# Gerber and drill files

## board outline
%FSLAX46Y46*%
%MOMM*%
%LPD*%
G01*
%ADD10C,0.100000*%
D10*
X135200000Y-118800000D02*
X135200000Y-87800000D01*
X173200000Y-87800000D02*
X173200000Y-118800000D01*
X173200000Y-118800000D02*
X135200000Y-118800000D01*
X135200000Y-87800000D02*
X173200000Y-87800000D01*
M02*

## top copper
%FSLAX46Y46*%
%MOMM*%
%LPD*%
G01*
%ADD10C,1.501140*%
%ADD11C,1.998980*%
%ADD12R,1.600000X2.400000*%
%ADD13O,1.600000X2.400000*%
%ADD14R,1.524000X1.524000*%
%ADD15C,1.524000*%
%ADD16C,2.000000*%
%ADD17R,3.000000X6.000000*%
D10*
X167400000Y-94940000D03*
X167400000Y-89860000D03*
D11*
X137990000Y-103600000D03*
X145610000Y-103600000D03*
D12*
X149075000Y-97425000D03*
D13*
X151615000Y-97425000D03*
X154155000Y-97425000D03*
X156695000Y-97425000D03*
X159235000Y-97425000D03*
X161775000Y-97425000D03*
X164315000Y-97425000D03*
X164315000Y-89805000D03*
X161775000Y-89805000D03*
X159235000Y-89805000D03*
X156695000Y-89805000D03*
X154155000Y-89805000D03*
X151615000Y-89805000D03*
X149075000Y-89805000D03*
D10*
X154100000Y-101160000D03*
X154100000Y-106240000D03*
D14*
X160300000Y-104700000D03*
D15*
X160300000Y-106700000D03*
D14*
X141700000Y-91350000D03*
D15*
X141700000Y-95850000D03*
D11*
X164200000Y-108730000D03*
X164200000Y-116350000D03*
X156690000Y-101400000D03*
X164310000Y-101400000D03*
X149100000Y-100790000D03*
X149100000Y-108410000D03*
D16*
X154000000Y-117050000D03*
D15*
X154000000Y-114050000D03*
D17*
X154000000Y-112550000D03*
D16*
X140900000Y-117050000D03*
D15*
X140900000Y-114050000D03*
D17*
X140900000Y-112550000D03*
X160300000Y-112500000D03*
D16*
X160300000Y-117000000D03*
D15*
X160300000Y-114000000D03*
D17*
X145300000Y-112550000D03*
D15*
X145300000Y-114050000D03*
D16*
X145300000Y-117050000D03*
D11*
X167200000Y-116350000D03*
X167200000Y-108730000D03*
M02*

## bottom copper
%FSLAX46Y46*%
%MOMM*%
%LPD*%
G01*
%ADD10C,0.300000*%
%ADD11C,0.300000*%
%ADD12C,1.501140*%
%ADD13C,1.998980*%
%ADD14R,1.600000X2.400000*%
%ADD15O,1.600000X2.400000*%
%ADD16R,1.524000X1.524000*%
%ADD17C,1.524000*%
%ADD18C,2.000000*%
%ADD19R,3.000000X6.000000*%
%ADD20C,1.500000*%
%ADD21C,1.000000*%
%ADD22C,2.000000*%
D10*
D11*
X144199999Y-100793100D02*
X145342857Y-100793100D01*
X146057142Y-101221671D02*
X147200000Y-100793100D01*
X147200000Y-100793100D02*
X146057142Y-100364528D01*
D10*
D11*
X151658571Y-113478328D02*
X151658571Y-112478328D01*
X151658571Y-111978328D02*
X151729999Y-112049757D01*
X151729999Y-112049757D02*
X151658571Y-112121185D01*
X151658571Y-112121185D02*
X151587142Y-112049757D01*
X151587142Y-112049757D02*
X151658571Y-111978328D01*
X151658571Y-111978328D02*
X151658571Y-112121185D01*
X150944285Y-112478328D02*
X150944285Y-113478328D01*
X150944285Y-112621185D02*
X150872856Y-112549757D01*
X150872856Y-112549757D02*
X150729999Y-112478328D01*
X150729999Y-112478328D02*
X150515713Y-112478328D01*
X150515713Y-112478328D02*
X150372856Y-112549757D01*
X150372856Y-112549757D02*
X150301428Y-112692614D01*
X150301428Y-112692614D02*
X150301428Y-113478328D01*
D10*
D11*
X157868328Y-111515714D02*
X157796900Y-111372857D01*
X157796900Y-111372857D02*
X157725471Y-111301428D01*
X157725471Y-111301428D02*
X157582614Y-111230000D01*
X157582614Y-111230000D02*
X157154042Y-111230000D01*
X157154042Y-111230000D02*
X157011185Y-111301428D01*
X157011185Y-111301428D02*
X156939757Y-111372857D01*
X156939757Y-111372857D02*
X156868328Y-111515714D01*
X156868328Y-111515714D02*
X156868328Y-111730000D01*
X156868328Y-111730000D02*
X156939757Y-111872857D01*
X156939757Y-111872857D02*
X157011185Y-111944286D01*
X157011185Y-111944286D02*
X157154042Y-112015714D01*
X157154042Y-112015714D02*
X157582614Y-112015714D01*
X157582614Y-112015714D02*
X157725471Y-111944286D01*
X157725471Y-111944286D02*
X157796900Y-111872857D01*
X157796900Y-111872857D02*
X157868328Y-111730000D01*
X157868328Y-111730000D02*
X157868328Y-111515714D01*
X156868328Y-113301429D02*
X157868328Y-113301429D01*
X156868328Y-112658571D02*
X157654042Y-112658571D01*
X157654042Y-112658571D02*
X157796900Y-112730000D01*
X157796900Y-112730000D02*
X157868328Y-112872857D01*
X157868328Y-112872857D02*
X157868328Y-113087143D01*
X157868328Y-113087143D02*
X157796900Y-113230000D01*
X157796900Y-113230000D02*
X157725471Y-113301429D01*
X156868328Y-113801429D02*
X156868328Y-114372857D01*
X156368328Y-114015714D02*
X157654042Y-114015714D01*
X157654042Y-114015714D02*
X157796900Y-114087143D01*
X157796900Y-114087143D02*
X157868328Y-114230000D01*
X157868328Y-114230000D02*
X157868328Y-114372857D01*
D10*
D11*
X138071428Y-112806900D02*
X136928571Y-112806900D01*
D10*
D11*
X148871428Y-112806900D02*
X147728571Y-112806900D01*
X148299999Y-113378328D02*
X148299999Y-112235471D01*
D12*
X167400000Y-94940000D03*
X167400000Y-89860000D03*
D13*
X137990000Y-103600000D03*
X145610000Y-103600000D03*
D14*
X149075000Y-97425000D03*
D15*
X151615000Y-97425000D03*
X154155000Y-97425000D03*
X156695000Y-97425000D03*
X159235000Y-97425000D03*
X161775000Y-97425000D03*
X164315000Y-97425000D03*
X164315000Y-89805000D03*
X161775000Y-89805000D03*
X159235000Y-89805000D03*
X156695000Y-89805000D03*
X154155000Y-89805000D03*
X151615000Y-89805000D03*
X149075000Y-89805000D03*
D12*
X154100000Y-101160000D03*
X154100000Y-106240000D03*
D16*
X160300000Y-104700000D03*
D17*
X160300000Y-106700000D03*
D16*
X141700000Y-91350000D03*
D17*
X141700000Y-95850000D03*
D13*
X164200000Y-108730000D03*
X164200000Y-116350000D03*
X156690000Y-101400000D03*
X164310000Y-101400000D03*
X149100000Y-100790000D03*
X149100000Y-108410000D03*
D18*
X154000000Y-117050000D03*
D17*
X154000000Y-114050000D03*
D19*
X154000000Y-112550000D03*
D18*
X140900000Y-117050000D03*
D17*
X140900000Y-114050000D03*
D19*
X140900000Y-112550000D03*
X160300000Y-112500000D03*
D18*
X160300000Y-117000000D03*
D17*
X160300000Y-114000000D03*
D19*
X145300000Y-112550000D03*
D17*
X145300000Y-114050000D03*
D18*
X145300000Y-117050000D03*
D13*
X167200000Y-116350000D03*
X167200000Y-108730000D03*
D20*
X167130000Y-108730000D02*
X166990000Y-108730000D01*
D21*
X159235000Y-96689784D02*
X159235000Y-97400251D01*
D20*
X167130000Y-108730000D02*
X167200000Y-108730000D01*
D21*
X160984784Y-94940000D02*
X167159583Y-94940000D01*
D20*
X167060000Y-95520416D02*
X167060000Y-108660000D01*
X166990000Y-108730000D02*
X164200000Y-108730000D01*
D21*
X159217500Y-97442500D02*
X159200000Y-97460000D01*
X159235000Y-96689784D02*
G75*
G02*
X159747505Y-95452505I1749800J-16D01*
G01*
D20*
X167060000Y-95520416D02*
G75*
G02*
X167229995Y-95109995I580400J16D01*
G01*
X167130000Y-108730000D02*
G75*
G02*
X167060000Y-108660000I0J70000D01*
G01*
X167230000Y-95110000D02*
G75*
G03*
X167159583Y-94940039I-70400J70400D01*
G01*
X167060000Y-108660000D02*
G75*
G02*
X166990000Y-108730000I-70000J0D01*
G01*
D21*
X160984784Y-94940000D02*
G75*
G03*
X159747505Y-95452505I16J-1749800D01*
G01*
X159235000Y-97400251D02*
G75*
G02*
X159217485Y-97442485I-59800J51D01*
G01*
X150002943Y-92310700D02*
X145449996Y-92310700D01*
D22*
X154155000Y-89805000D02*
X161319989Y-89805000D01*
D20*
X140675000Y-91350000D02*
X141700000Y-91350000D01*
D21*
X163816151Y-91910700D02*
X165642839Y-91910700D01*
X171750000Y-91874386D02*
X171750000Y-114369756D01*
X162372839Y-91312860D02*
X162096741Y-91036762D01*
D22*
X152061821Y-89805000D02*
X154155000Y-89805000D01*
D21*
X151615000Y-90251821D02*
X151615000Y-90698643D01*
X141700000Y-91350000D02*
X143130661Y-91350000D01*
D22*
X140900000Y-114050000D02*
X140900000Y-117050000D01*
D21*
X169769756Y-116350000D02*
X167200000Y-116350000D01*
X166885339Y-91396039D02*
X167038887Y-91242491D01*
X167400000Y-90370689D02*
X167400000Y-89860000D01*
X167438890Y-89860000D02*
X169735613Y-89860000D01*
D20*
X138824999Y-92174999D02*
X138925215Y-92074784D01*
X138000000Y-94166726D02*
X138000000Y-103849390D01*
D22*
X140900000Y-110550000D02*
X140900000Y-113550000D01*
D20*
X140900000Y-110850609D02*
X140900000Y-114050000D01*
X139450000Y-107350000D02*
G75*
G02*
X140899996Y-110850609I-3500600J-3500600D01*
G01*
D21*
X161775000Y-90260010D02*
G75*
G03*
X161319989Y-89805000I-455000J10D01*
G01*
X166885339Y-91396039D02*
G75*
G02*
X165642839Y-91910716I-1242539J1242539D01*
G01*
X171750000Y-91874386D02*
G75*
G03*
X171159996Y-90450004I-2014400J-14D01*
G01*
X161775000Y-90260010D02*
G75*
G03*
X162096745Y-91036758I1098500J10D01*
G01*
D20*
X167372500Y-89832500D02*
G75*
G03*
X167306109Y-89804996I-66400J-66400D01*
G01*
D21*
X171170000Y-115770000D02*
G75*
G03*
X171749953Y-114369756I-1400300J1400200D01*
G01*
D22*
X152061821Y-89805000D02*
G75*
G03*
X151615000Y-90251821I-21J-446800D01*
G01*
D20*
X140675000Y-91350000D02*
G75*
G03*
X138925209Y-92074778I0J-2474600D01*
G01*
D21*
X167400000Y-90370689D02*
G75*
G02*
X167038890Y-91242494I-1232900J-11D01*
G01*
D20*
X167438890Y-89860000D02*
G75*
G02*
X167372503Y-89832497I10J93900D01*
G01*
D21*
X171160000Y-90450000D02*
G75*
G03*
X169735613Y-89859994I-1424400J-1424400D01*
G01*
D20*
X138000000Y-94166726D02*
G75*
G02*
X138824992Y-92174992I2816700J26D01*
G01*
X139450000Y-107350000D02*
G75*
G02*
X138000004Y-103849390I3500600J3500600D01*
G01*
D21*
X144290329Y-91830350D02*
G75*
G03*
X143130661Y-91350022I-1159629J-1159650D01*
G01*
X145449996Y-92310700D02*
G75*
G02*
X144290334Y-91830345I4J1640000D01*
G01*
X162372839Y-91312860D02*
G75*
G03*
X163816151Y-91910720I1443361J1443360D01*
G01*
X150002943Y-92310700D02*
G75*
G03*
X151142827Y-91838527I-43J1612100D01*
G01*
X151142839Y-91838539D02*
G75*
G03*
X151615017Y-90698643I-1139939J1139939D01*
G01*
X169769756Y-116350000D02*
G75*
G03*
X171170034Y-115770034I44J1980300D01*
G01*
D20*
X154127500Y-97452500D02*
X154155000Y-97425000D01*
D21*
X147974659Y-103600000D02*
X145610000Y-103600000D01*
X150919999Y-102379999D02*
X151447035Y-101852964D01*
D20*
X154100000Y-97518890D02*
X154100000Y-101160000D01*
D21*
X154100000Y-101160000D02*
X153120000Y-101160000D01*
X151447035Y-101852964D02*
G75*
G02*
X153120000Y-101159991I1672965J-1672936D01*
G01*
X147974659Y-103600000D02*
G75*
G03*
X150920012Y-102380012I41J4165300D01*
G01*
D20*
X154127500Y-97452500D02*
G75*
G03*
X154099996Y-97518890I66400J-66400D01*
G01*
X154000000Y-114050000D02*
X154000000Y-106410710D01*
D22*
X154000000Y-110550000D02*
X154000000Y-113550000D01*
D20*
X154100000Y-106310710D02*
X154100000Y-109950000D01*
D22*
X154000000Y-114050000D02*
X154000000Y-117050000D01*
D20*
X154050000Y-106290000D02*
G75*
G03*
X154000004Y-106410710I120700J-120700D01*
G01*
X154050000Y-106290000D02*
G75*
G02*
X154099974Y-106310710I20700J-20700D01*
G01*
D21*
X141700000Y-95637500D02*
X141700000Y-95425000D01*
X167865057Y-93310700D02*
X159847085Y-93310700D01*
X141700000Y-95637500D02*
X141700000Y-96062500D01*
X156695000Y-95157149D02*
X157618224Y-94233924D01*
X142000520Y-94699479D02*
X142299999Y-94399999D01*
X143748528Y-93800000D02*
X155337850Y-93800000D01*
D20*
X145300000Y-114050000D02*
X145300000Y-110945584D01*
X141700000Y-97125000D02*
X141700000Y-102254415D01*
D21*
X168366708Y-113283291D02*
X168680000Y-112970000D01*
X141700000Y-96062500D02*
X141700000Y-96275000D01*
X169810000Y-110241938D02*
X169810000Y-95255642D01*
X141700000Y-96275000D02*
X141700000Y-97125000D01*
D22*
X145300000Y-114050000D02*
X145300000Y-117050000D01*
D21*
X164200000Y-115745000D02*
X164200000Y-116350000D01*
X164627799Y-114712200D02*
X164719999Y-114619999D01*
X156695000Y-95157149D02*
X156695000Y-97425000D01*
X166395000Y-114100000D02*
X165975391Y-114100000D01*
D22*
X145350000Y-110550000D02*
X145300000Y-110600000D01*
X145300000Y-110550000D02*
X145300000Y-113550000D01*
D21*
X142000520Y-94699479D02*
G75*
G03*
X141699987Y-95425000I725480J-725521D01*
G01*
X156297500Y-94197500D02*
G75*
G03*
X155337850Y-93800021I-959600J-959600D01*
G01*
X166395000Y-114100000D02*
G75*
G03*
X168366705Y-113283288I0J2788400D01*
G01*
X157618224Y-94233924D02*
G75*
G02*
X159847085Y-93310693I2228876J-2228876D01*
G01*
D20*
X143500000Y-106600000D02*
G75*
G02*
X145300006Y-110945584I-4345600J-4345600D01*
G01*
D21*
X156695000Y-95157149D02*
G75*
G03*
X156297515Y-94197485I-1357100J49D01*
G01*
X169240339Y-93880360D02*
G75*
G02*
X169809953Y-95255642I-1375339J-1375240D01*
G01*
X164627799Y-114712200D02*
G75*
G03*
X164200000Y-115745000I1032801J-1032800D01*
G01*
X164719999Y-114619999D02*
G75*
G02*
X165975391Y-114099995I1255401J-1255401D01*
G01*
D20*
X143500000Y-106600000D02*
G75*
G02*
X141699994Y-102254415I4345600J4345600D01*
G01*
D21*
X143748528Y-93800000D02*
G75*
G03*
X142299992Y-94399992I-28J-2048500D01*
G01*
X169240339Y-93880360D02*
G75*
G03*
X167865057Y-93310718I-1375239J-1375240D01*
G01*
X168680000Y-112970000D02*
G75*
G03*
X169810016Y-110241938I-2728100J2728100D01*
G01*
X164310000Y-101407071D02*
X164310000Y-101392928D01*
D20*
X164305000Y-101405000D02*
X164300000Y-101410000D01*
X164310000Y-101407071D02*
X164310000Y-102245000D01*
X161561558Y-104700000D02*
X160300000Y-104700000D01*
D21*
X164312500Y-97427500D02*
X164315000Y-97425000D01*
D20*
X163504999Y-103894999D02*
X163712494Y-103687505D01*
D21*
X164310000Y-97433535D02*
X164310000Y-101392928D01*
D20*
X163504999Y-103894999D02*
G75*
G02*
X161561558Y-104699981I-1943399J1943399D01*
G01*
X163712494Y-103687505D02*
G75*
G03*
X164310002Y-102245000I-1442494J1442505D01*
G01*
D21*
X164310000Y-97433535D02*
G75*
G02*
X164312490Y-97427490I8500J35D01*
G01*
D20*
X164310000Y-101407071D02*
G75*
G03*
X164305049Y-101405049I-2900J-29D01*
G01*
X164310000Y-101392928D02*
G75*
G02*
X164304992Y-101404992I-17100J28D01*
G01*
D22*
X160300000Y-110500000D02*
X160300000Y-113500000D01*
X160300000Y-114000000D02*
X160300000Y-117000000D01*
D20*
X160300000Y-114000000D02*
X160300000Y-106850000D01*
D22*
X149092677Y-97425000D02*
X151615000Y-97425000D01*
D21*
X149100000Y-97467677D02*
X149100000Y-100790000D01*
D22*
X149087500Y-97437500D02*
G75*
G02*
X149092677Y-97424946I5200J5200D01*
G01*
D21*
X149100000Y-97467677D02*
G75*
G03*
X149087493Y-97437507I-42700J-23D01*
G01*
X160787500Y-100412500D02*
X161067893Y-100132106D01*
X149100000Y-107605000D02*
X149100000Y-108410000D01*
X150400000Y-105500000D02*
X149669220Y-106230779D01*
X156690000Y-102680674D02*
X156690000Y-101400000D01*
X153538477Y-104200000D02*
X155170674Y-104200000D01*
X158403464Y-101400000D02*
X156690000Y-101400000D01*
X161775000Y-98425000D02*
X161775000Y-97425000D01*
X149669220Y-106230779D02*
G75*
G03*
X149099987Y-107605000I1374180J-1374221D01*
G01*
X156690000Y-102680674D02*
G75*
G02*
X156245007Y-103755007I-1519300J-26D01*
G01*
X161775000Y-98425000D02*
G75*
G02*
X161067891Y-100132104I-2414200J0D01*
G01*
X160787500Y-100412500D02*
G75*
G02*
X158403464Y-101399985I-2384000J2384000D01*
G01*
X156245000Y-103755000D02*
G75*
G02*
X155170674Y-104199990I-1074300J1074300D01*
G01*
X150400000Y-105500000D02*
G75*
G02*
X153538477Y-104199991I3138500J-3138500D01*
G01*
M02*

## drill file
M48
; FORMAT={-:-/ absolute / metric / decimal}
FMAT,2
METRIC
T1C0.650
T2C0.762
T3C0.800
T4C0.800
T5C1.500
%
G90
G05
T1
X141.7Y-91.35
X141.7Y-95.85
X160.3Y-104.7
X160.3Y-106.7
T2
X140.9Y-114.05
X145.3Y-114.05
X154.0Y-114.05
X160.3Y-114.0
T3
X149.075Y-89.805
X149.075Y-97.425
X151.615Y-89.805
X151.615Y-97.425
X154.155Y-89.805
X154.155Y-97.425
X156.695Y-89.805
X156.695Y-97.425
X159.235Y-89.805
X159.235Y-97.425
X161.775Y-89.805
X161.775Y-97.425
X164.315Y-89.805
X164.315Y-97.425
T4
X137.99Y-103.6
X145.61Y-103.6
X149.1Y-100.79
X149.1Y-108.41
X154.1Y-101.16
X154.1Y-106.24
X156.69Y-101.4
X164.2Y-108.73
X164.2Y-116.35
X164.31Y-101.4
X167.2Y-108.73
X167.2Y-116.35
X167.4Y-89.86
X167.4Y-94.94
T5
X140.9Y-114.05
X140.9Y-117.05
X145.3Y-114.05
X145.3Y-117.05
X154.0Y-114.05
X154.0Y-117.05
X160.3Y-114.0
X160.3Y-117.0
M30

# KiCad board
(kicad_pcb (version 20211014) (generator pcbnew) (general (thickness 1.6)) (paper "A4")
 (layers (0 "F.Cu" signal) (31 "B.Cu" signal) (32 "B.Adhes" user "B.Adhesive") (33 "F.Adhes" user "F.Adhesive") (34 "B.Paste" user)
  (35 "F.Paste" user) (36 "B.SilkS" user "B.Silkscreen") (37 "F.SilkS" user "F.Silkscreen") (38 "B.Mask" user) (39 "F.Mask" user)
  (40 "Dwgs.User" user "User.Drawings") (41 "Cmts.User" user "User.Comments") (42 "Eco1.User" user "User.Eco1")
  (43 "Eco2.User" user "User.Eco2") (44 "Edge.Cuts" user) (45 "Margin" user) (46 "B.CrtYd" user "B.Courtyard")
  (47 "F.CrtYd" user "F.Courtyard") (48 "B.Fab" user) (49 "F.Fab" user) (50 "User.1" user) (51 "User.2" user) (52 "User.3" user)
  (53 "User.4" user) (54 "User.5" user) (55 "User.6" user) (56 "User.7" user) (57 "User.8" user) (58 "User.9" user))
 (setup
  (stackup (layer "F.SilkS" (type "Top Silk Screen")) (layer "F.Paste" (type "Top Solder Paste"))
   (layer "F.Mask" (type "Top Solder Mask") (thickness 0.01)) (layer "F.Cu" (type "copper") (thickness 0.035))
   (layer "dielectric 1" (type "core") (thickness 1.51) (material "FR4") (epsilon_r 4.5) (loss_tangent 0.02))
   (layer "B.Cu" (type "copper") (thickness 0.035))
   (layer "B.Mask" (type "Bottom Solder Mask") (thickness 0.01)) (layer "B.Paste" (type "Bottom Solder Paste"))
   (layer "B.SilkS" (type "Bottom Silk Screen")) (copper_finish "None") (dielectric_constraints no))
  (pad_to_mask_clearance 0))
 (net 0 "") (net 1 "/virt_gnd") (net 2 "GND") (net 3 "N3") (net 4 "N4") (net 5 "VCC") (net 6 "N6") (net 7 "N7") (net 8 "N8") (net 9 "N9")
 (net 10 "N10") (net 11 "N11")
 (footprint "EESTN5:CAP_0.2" (layer "F.Cu") (at 167.4 92.4 90)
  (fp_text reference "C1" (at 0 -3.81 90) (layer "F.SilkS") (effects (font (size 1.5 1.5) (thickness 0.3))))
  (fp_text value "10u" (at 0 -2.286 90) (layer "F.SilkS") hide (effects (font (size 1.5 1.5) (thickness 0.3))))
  (pad "1" thru_hole circle locked (at -2.54 0 90) (size 1.50114 1.50114) (drill 0.8001) (layers *.Cu *.Mask "F.SilkS") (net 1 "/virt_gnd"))
  (pad "2" thru_hole circle locked (at 2.54 0 90) (size 1.50114 1.50114) (drill 0.8001) (layers *.Cu *.Mask "F.SilkS") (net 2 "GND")))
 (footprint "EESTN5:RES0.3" (layer "F.Cu") (at 141.8 103.6) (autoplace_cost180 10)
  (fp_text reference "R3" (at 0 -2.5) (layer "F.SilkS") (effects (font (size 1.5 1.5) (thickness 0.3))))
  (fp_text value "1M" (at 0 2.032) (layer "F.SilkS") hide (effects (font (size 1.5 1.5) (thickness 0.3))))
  (pad "1" thru_hole circle (at -3.81 0) (size 1.99898 1.99898) (drill 0.8001) (layers *.Cu *.Mask "F.SilkS") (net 2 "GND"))
  (pad "2" thru_hole circle (at 3.81 0) (size 1.99898 1.99898) (drill 0.8001) (layers *.Cu *.Mask "F.SilkS") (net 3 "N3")))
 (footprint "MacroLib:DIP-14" (layer "F.Cu") (at 149.075 97.425 90)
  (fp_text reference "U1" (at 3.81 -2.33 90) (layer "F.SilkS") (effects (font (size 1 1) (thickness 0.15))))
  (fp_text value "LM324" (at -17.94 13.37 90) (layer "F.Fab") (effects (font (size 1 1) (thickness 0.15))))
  (pad "1" thru_hole rect (at 0 0 90) (size 2.4 1.6) (drill 0.8) (layers *.Cu *.Mask) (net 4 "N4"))
  (pad "2" thru_hole oval (at 0 2.54 90) (size 2.4 1.6) (drill 0.8) (layers *.Cu *.Mask) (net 4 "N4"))
  (pad "3" thru_hole oval (at 0 5.08 90) (size 2.4 1.6) (drill 0.8) (layers *.Cu *.Mask) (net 3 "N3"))
  (pad "4" thru_hole oval (at 0 7.62 90) (size 2.4 1.6) (drill 0.8) (layers *.Cu *.Mask) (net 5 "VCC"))
  (pad "5" thru_hole oval (at 0 10.16 90) (size 2.4 1.6) (drill 0.8) (layers *.Cu *.Mask) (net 1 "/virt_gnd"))
  (pad "6" thru_hole oval (at 0 12.7 90) (size 2.4 1.6) (drill 0.8) (layers *.Cu *.Mask) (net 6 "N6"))
  (pad "7" thru_hole oval (at 0 15.24 90) (size 2.4 1.6) (drill 0.8) (layers *.Cu *.Mask) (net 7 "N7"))
  (pad "8" thru_hole oval (at 7.62 15.24 90) (size 2.4 1.6) (drill 0.8) (layers *.Cu *.Mask) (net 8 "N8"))
  (pad "9" thru_hole oval (at 7.62 12.7 90) (size 2.4 1.6) (drill 0.8) (layers *.Cu *.Mask) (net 2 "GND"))
  (pad "10" thru_hole oval (at 7.62 10.16 90) (size 2.4 1.6) (drill 0.8) (layers *.Cu *.Mask) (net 2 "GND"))
  (pad "11" thru_hole oval (at 7.62 7.62 90) (size 2.4 1.6) (drill 0.8) (layers *.Cu *.Mask) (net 2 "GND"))
  (pad "12" thru_hole oval (at 7.62 5.08 90) (size 2.4 1.6) (drill 0.8) (layers *.Cu *.Mask) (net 2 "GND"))
  (pad "13" thru_hole oval (at 7.62 2.54 90) (size 2.4 1.6) (drill 0.8) (layers *.Cu *.Mask) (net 2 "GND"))
  (pad "14" thru_hole oval (at 7.62 0 90) (size 2.4 1.6) (drill 0.8) (layers *.Cu *.Mask) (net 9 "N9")))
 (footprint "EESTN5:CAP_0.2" (layer "F.Cu") (at 154.1 103.7 -90)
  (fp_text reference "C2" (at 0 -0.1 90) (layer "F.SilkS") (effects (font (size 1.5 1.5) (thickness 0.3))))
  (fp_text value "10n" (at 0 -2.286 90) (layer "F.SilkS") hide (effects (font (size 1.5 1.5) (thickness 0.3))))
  (pad "1" thru_hole circle locked (at -2.54 0 270) (size 1.50114 1.50114) (drill 0.8001) (layers *.Cu *.Mask "F.SilkS") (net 3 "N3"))
  (pad "2" thru_hole circle locked (at 2.54 0 270) (size 1.50114 1.50114) (drill 0.8001) (layers *.Cu *.Mask "F.SilkS") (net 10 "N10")))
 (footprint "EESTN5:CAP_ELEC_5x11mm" (layer "F.Cu") (at 160.3 105.7 180)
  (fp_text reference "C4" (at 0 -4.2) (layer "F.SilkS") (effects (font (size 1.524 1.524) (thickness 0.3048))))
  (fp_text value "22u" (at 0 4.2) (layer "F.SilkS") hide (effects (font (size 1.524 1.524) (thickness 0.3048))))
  (pad "1" thru_hole rect locked (at 0 1 180) (size 1.524 1.524) (drill 0.65) (layers *.Cu *.Mask "F.SilkS") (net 7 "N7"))
  (pad "2" thru_hole circle locked (at 0 -1 180) (size 1.524 1.524) (drill 0.65) (layers *.Cu *.Mask "F.SilkS") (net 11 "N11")))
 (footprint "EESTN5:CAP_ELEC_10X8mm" (layer "F.Cu") (at 141.7 93.6 180)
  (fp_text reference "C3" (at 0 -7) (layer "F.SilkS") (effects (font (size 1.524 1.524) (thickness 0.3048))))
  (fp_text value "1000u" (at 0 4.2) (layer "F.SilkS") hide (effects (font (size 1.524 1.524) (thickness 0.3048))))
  (pad "1" thru_hole rect locked (at 0 2.25 180) (size 1.524 1.524) (drill 0.65) (layers *.Cu *.Mask "F.SilkS") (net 2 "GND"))
  (pad "2" thru_hole circle locked (at 0 -2.25 180) (size 1.524 1.524) (drill 0.65) (layers *.Cu *.Mask "F.SilkS") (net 5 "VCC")))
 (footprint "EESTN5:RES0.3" (layer "F.Cu") (at 164.2 112.54 -90) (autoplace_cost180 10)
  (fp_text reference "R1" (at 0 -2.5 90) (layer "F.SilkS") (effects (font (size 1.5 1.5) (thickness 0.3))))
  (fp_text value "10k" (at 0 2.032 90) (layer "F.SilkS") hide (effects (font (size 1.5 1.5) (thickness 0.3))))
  (pad "1" thru_hole circle (at -3.81 0 270) (size 1.99898 1.99898) (drill 0.8001) (layers *.Cu *.Mask "F.SilkS") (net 1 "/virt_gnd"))
  (pad "2" thru_hole circle (at 3.81 0 270) (size 1.99898 1.99898) (drill 0.8001) (layers *.Cu *.Mask "F.SilkS") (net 5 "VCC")))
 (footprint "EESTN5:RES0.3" (layer "F.Cu") (at 160.5 101.4) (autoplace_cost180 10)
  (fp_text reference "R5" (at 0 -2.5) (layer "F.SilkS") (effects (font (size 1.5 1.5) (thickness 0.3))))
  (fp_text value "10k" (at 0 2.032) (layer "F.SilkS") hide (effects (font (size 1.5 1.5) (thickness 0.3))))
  (pad "1" thru_hole circle (at -3.81 0) (size 1.99898 1.99898) (drill 0.8001) (layers *.Cu *.Mask "F.SilkS") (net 6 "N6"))
  (pad "2" thru_hole circle (at 3.81 0) (size 1.99898 1.99898) (drill 0.8001) (layers *.Cu *.Mask "F.SilkS") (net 7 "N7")))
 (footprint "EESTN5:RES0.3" (layer "F.Cu") (at 149.1 104.6 -90) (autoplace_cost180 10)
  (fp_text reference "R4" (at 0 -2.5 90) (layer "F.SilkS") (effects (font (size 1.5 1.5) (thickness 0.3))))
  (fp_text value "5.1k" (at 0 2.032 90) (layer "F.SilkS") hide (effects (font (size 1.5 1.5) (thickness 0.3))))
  (pad "1" thru_hole circle (at -3.81 0 270) (size 1.99898 1.99898) (drill 0.8001) (layers *.Cu *.Mask "F.SilkS") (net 4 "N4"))
  (pad "2" thru_hole circle (at 3.81 0 270) (size 1.99898 1.99898) (drill 0.8001) (layers *.Cu *.Mask "F.SilkS") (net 6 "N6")))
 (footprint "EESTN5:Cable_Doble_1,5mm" (layer "F.Cu") (at 154 114.05 180)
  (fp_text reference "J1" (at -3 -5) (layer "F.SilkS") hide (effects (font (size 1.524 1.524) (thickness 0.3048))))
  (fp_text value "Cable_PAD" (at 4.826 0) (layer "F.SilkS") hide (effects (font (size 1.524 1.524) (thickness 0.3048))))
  (pad "1" thru_hole circle locked (at 0 -3 180) (size 2 2) (drill 1.5) (layers *.Cu *.Mask) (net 10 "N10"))
  (pad "1" thru_hole circle locked (at 0 0 180) (size 1.524 1.524) (drill 0.762) (layers *.Cu *.Mask) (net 10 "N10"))
  (pad "1" thru_hole rect locked (at 0 0 180) (size 3 6) (drill 1.5 (offset 0 1.5)) (layers *.Cu "F.SilkS") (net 10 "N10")))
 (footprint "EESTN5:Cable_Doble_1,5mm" (layer "F.Cu") (at 140.9 114.05 180)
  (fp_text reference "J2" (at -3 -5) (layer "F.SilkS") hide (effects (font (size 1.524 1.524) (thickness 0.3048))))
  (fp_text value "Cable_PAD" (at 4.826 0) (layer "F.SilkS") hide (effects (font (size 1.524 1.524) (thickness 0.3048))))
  (pad "1" thru_hole circle locked (at 0 -3 180) (size 2 2) (drill 1.5) (layers *.Cu *.Mask) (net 2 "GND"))
  (pad "1" thru_hole circle locked (at 0 0 180) (size 1.524 1.524) (drill 0.762) (layers *.Cu *.Mask) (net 2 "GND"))
  (pad "1" thru_hole rect locked (at 0 0 180) (size 3 6) (drill 1.5 (offset 0 1.5)) (layers *.Cu "F.SilkS") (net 2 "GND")))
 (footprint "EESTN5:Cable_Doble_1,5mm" (layer "F.Cu") (at 160.3 114 180)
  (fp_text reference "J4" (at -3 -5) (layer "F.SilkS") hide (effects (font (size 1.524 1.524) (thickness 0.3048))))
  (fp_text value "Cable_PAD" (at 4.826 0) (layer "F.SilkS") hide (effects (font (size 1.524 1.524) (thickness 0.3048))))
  (pad "1" thru_hole rect locked (at 0 0 180) (size 3 6) (drill 1.5 (offset 0 1.5)) (layers *.Cu "F.SilkS") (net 11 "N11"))
  (pad "1" thru_hole circle locked (at 0 -3 180) (size 2 2) (drill 1.5) (layers *.Cu *.Mask) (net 11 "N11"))
  (pad "1" thru_hole circle locked (at 0 0 180) (size 1.524 1.524) (drill 0.762) (layers *.Cu *.Mask) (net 11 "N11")))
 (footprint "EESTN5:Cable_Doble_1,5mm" (layer "F.Cu") (at 145.3 114.05 180)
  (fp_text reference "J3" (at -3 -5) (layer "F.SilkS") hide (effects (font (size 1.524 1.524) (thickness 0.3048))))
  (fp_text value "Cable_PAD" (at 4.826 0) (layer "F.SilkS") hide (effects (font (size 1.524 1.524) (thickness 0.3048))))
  (pad "1" thru_hole rect locked (at 0 0 180) (size 3 6) (drill 1.5 (offset 0 1.5)) (layers *.Cu "F.SilkS") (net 5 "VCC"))
  (pad "1" thru_hole circle locked (at 0 0 180) (size 1.524 1.524) (drill 0.762) (layers *.Cu *.Mask) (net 5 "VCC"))
  (pad "1" thru_hole circle locked (at 0 -3 180) (size 2 2) (drill 1.5) (layers *.Cu *.Mask) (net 5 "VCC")))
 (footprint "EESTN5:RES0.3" (layer "F.Cu") (at 167.2 112.54 90) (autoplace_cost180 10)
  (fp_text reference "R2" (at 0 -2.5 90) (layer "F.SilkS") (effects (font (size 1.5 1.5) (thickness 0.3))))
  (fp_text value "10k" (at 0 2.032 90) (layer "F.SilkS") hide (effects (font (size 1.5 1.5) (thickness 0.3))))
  (pad "1" thru_hole circle (at -3.81 0 90) (size 1.99898 1.99898) (drill 0.8001) (layers *.Cu *.Mask "F.SilkS") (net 2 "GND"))
  (pad "2" thru_hole circle (at 3.81 0 90) (size 1.99898 1.99898) (drill 0.8001) (layers *.Cu *.Mask "F.SilkS") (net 1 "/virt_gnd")))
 (gr_line (start 135.2 118.8) (end 135.2 87.8) (layer "Edge.Cuts") (width 0.1))
 (gr_line (start 173.2 87.8) (end 173.2 118.8) (layer "Edge.Cuts") (width 0.1))
 (gr_line (start 173.2 118.8) (end 135.2 118.8) (layer "Edge.Cuts") (width 0.1))
 (gr_line (start 135.2 87.8) (end 173.2 87.8) (layer "Edge.Cuts") (width 0.1))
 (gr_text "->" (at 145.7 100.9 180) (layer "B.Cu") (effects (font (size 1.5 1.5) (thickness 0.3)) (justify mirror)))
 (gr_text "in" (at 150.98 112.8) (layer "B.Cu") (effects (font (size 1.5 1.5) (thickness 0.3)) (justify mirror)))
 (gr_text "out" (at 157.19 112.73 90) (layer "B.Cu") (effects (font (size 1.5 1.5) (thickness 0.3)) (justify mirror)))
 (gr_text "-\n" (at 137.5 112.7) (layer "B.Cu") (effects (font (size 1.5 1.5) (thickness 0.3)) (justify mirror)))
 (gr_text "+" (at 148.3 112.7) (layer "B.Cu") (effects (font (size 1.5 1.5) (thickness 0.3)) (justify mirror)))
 (segment (start 167.13 108.73) (end 166.99 108.73) (width 1.5) (layer "B.Cu") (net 1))
 (segment (start 159.235 96.689784) (end 159.235 97.400251) (width 1) (layer "B.Cu") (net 1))
 (segment (start 167.13 108.73) (end 167.2 108.73) (width 1.5) (layer "B.Cu") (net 1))
 (segment (start 160.984784 94.94) (end 167.159583 94.94) (width 1) (layer "B.Cu") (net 1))
 (segment (start 167.06 95.520416) (end 167.06 108.66) (width 1.5) (layer "B.Cu") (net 1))
 (segment (start 166.99 108.73) (end 164.2 108.73) (width 1.5) (layer "B.Cu") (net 1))
 (segment (start 159.2175 97.4425) (end 159.2 97.46) (width 1) (layer "B.Cu") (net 1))
 (arc (start 159.235 96.689784) (mid 159.368194 96.02017) (end 159.7475 95.4525) (width 1) (layer "B.Cu") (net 1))
 (arc (start 167.06 95.520416) (mid 167.104181 95.2983) (end 167.23 95.11) (width 1.5) (layer "B.Cu") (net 1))
 (arc (start 167.13 108.73) (mid 167.080502 108.709497) (end 167.06 108.66) (width 1.5) (layer "B.Cu") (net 1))
 (arc (start 167.23 95.11) (mid 167.251586 95.001474) (end 167.159583 94.94) (width 1.5) (layer "B.Cu") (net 1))
 (arc (start 167.06 108.66) (mid 167.039497 108.709497) (end 166.99 108.73) (width 1.5) (layer "B.Cu") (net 1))
 (arc (start 160.984784 94.94) (mid 160.31517 95.073194) (end 159.7475 95.4525) (width 1) (layer "B.Cu") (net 1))
 (arc (start 159.235 97.400251) (mid 159.230451 97.423116) (end 159.2175 97.4425) (width 1) (layer "B.Cu") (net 1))
 (segment (start 150.002943 92.3107) (end 145.449996 92.3107) (width 1) (layer "B.Cu") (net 2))
 (segment (start 154.155 89.805) (end 161.319989 89.805) (width 2) (layer "B.Cu") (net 2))
 (segment (start 140.675 91.35) (end 141.7 91.35) (width 1.5) (layer "B.Cu") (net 2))
 (segment (start 163.816151 91.9107) (end 165.642839 91.9107) (width 1) (layer "B.Cu") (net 2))
 (segment (start 171.75 91.874386) (end 171.75 114.369756) (width 1) (layer "B.Cu") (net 2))
 (segment (start 162.372839 91.31286) (end 162.096741 91.036762) (width 1) (layer "B.Cu") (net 2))
 (segment (start 152.061821 89.805) (end 154.155 89.805) (width 2) (layer "B.Cu") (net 2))
 (segment (start 151.615 90.251821) (end 151.615 90.698643) (width 1) (layer "B.Cu") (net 2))
 (segment (start 141.7 91.35) (end 143.130661 91.35) (width 1) (layer "B.Cu") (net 2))
 (segment (start 140.9 114.05) (end 140.9 117.05) (width 2) (layer "B.Cu") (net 2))
 (segment (start 169.769756 116.35) (end 167.2 116.35) (width 1) (layer "B.Cu") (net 2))
 (segment (start 166.885339 91.396039) (end 167.038887 91.242491) (width 1) (layer "B.Cu") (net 2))
 (segment (start 167.4 90.370689) (end 167.4 89.86) (width 1) (layer "B.Cu") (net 2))
 (segment (start 167.43889 89.86) (end 169.735613 89.86) (width 1) (layer "B.Cu") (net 2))
 (segment (start 138.824999 92.174999) (end 138.925215 92.074784) (width 1.5) (layer "B.Cu") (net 2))
 (segment (start 138 94.166726) (end 138 103.84939) (width 1.5) (layer "B.Cu") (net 2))
 (segment (start 140.9 110.55) (end 140.9 113.55) (width 2) (layer "B.Cu") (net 2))
 (segment (start 140.9 110.850609) (end 140.9 114.05) (width 1.5) (layer "B.Cu") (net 2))
 (arc (start 139.45 107.35) (mid 140.523157 108.956093) (end 140.9 110.850609) (width 1.5) (layer "B.Cu") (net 2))
 (arc (start 161.775 90.26001) (mid 161.64173 89.938269) (end 161.319989 89.805) (width 1) (layer "B.Cu") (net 2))
 (arc (start 166.885339 91.396039) (mid 166.315275 91.776943) (end 165.642839 91.9107) (width 1) (layer "B.Cu") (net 2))
 (arc (start 171.75 91.874386) (mid 171.596663 91.103513) (end 171.16 90.45) (width 1) (layer "B.Cu") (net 2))
 (arc (start 161.775 90.26001) (mid 161.858617 90.680385) (end 162.096741 91.036762) (width 1) (layer "B.Cu") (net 2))
 (arc (start 167.3725 89.8325) (mid 167.342039 89.812147) (end 167.306109 89.805) (width 1.5) (layer "B.Cu") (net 2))
 (arc (start 171.17 115.77) (mid 171.599262 115.127562) (end 171.75 114.369756) (width 1) (layer "B.Cu") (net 2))
 (arc (start 152.061821 89.805) (mid 151.74587 89.93587) (end 151.615 90.251821) (width 2) (layer "B.Cu") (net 2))
 (arc (start 140.675 91.35) (mid 139.728023 91.538365) (end 138.925215 92.074784) (width 1.5) (layer "B.Cu") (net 2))
 (arc (start 167.4 90.370689) (mid 167.306149 90.842504) (end 167.038887 91.242491) (width 1) (layer "B.Cu") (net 2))
 (arc (start 167.43889 89.86) (mid 167.40296 89.852852) (end 167.3725 89.8325) (width 1.5) (layer "B.Cu") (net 2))
 (arc (start 171.16 90.45) (mid 170.506485 90.013336) (end 169.735613 89.86) (width 1) (layer "B.Cu") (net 2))
 (arc (start 138 94.166726) (mid 138.21441 93.088811) (end 138.824999 92.174999) (width 1.5) (layer "B.Cu") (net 2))
 (arc (start 139.45 107.35) (mid 138.376842 105.743906) (end 138 103.84939) (width 1.5) (layer "B.Cu") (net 2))
 (arc (start 144.290329 91.83035) (mid 143.758268 91.474838) (end 143.130661 91.35) (width 1) (layer "B.Cu") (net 2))
 (arc (start 145.449996 92.3107) (mid 144.822388 92.185861) (end 144.290329 91.83035) (width 1) (layer "B.Cu") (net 2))
 (arc (start 162.372839 91.31286) (mid 163.035036 91.755326) (end 163.816151 91.9107) (width 1) (layer "B.Cu") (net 2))
 (arc (start 150.002943 92.3107) (mid 150.61985 92.187989) (end 151.142839 91.838539) (width 1) (layer "B.Cu") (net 2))
 (arc (start 151.142839 91.838539) (mid 151.492289 91.31555) (end 151.615 90.698643) (width 1) (layer "B.Cu") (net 2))
 (arc (start 169.769756 116.35) (mid 170.527562 116.199262) (end 171.17 115.77) (width 1) (layer "B.Cu") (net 2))
 (segment (start 154.1275 97.4525) (end 154.155 97.425) (width 1.5) (layer "B.Cu") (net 3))
 (segment (start 147.974659 103.6) (end 145.61 103.6) (width 1) (layer "B.Cu") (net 3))
 (segment (start 150.919999 102.379999) (end 151.447035 101.852964) (width 1) (layer "B.Cu") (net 3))
 (segment (start 154.1 97.51889) (end 154.1 101.16) (width 1.5) (layer "B.Cu") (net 3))
 (segment (start 154.1 101.16) (end 153.12 101.16) (width 1) (layer "B.Cu") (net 3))
 (arc (start 151.447035 101.852964) (mid 152.214597 101.340095) (end 153.12 101.16) (width 1) (layer "B.Cu") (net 3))
 (arc (start 147.974659 103.6) (mid 149.568665 103.282932) (end 150.919999 102.379999) (width 1) (layer "B.Cu") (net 3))
 (arc (start 154.1275 97.4525) (mid 154.107147 97.48296) (end 154.1 97.51889) (width 1.5) (layer "B.Cu") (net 3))
 (segment (start 154 114.05) (end 154 106.41071) (width 1.5) (layer "B.Cu") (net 10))
 (segment (start 154 110.55) (end 154 113.55) (width 2) (layer "B.Cu") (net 10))
 (segment (start 154.1 106.31071) (end 154.1 109.95) (width 1.5) (layer "B.Cu") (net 10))
 (segment (start 154 114.05) (end 154 117.05) (width 2) (layer "B.Cu") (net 10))
 (arc (start 154.05 106.29) (mid 154.012994 106.345382) (end 154 106.41071) (width 1.5) (layer "B.Cu") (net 10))
 (arc (start 154.05 106.29) (mid 154.081919 106.28365) (end 154.1 106.31071) (width 1.5) (layer "B.Cu") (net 10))
 (segment (start 141.7 95.6375) (end 141.7 95.425) (width 1) (layer "B.Cu") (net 5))
 (segment (start 167.865057 93.3107) (end 159.847085 93.3107) (width 1) (layer "B.Cu") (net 5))
 (segment (start 141.7 95.6375) (end 141.7 96.0625) (width 1) (layer "B.Cu") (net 5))
 (segment (start 156.695 95.157149) (end 157.618224 94.233924) (width 1) (layer "B.Cu") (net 5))
 (segment (start 142.00052 94.699479) (end 142.299999 94.399999) (width 1) (layer "B.Cu") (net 5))
 (segment (start 143.748528 93.8) (end 155.33785 93.8) (width 1) (layer "B.Cu") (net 5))
 (segment (start 145.3 114.05) (end 145.3 110.945584) (width 1.5) (layer "B.Cu") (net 5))
 (segment (start 141.7 97.125) (end 141.7 102.254415) (width 1.5) (layer "B.Cu") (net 5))
 (segment (start 168.366708 113.283291) (end 168.68 112.97) (width 1) (layer "B.Cu") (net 5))
 (segment (start 141.7 96.0625) (end 141.7 96.275) (width 1) (layer "B.Cu") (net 5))
 (segment (start 169.81 110.241938) (end 169.81 95.255642) (width 1) (layer "B.Cu") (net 5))
 (segment (start 141.7 96.275) (end 141.7 97.125) (width 1) (layer "B.Cu") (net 5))
 (segment (start 145.3 114.05) (end 145.3 117.05) (width 2) (layer "B.Cu") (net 5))
 (segment (start 164.2 115.745) (end 164.2 116.35) (width 1) (layer "B.Cu") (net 5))
 (segment (start 164.627799 114.7122) (end 164.719999 114.619999) (width 1) (layer "B.Cu") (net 5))
 (segment (start 156.695 95.157149) (end 156.695 97.425) (width 1) (layer "B.Cu") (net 5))
 (segment (start 166.395 114.1) (end 165.975391 114.1) (width 1) (layer "B.Cu") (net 5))
 (segment (start 145.35 110.55) (end 145.3 110.6) (width 2) (layer "B.Cu") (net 5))
 (segment (start 145.3 110.55) (end 145.3 113.55) (width 2) (layer "B.Cu") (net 5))
 (arc (start 142.00052 94.699479) (mid 141.778102 95.032351) (end 141.7 95.425) (width 1) (layer "B.Cu") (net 5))
 (arc (start 156.2975 94.1975) (mid 155.857208 93.903306) (end 155.33785 93.8) (width 1) (layer "B.Cu") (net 5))
 (arc (start 166.395 114.1) (mid 167.46208 113.887744) (end 168.366708 113.283291) (width 1) (layer "B.Cu") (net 5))
 (arc (start 157.618224 94.233924) (mid 158.640834 93.550638) (end 159.847085 93.3107) (width 1) (layer "B.Cu") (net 5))
 (arc (start 143.5 106.6) (mid 144.832195 108.59377) (end 145.3 110.945584) (width 1.5) (layer "B.Cu") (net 5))
 (arc (start 156.695 95.157149) (mid 156.591693 94.63779) (end 156.2975 94.1975) (width 1) (layer "B.Cu") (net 5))
 (arc (start 169.240339 93.88036) (mid 169.661949 94.511345) (end 169.81 95.255642) (width 1) (layer "B.Cu") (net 5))
 (arc (start 164.627799 114.7122) (mid 164.311181 115.186052) (end 164.2 115.745) (width 1) (layer "B.Cu") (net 5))
 (arc (start 164.719999 114.619999) (mid 165.295978 114.235143) (end 165.975391 114.1) (width 1) (layer "B.Cu") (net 5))
 (arc (start 143.5 106.6) (mid 142.167804 104.606228) (end 141.7 102.254415) (width 1.5) (layer "B.Cu") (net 5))
 (arc (start 143.748528 93.8) (mid 142.96459 93.955934) (end 142.299999 94.399999) (width 1) (layer "B.Cu") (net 5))
 (arc (start 169.240339 93.88036) (mid 168.609354 93.458749) (end 167.865057 93.3107) (width 1) (layer "B.Cu") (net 5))
 (arc (start 168.68 112.97) (mid 169.516322 111.718354) (end 169.81 110.241938) (width 1) (layer "B.Cu") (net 5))
 (segment (start 164.31 101.407071) (end 164.31 101.392928) (width 1) (layer "B.Cu") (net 7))
 (segment (start 164.305 101.405) (end 164.3 101.41) (width 1.5) (layer "B.Cu") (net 7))
 (segment (start 164.31 101.407071) (end 164.31 102.245) (width 1.5) (layer "B.Cu") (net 7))
 (segment (start 161.561558 104.7) (end 160.3 104.7) (width 1.5) (layer "B.Cu") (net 7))
 (segment (start 164.3125 97.4275) (end 164.315 97.425) (width 1) (layer "B.Cu") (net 7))
 (segment (start 163.504999 103.894999) (end 163.712494 103.687505) (width 1.5) (layer "B.Cu") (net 7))
 (segment (start 164.31 97.433535) (end 164.31 101.392928) (width 1) (layer "B.Cu") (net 7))
 (arc (start 163.504999 103.894999) (mid 162.61334 104.490787) (end 161.561558 104.7) (width 1.5) (layer "B.Cu") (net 7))
 (arc (start 163.712494 103.687505) (mid 164.154713 103.025678) (end 164.31 102.245) (width 1.5) (layer "B.Cu") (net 7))
 (arc (start 164.31 97.433535) (mid 164.310649 97.430268) (end 164.3125 97.4275) (width 1) (layer "B.Cu") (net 7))
 (arc (start 164.31 101.407071) (mid 164.308191 101.404365) (end 164.305 101.405) (width 1.5) (layer "B.Cu") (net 7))
 (arc (start 164.31 101.392928) (mid 164.3087 101.399461) (end 164.305 101.405) (width 1.5) (layer "B.Cu") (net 7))
 (segment (start 160.3 110.5) (end 160.3 113.5) (width 2) (layer "B.Cu") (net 11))
 (segment (start 160.3 114) (end 160.3 117) (width 2) (layer "B.Cu") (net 11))
 (segment (start 160.3 114) (end 160.3 106.85) (width 1.5) (layer "B.Cu") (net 11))
 (segment (start 149.092677 97.425) (end 151.615 97.425) (width 2) (layer "B.Cu") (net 4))
 (segment (start 149.1 97.467677) (end 149.1 100.79) (width 1) (layer "B.Cu") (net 4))
 (arc (start 149.0875 97.4375) (mid 149.085912 97.42952) (end 149.092677 97.425) (width 2) (layer "B.Cu") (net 4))
 (arc (start 149.1 97.467677) (mid 149.096751 97.451345) (end 149.0875 97.4375) (width 1) (layer "B.Cu") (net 4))
 (segment (start 160.7875 100.4125) (end 161.067893 100.132106) (width 1) (layer "B.Cu") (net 6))
 (segment (start 149.1 107.605) (end 149.1 108.41) (width 1) (layer "B.Cu") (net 6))
 (segment (start 150.4 105.5) (end 149.66922 106.230779) (width 1) (layer "B.Cu") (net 6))
 (segment (start 156.69 102.680674) (end 156.69 101.4) (width 1) (layer "B.Cu") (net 6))
 (segment (start 153.538477 104.2) (end 155.170674 104.2) (width 1) (layer "B.Cu") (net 6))
 (segment (start 158.403464 101.4) (end 156.69 101.4) (width 1) (layer "B.Cu") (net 6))
 (segment (start 161.775 98.425) (end 161.775 97.425) (width 1) (layer "B.Cu") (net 6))
 (arc (start 149.66922 106.230779) (mid 149.247935 106.861276) (end 149.1 107.605) (width 1) (layer "B.Cu") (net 6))
 (arc (start 156.69 102.680674) (mid 156.574348 103.262095) (end 156.245 103.755) (width 1) (layer "B.Cu") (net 6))
 (arc (start 161.775 98.425) (mid 161.591228 99.348879) (end 161.067893 100.132106) (width 1) (layer "B.Cu") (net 6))
 (arc (start 160.7875 100.4125) (mid 159.693695 101.143357) (end 158.403464 101.4) (width 1) (layer "B.Cu") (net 6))
 (arc (start 156.245 103.755) (mid 155.752095 104.084348) (end 155.170674 104.2) (width 1) (layer "B.Cu") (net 6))
 (arc (start 150.4 105.5) (mid 151.839945 104.537858) (end 153.538477 104.2) (width 1) (layer "B.Cu") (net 6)))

